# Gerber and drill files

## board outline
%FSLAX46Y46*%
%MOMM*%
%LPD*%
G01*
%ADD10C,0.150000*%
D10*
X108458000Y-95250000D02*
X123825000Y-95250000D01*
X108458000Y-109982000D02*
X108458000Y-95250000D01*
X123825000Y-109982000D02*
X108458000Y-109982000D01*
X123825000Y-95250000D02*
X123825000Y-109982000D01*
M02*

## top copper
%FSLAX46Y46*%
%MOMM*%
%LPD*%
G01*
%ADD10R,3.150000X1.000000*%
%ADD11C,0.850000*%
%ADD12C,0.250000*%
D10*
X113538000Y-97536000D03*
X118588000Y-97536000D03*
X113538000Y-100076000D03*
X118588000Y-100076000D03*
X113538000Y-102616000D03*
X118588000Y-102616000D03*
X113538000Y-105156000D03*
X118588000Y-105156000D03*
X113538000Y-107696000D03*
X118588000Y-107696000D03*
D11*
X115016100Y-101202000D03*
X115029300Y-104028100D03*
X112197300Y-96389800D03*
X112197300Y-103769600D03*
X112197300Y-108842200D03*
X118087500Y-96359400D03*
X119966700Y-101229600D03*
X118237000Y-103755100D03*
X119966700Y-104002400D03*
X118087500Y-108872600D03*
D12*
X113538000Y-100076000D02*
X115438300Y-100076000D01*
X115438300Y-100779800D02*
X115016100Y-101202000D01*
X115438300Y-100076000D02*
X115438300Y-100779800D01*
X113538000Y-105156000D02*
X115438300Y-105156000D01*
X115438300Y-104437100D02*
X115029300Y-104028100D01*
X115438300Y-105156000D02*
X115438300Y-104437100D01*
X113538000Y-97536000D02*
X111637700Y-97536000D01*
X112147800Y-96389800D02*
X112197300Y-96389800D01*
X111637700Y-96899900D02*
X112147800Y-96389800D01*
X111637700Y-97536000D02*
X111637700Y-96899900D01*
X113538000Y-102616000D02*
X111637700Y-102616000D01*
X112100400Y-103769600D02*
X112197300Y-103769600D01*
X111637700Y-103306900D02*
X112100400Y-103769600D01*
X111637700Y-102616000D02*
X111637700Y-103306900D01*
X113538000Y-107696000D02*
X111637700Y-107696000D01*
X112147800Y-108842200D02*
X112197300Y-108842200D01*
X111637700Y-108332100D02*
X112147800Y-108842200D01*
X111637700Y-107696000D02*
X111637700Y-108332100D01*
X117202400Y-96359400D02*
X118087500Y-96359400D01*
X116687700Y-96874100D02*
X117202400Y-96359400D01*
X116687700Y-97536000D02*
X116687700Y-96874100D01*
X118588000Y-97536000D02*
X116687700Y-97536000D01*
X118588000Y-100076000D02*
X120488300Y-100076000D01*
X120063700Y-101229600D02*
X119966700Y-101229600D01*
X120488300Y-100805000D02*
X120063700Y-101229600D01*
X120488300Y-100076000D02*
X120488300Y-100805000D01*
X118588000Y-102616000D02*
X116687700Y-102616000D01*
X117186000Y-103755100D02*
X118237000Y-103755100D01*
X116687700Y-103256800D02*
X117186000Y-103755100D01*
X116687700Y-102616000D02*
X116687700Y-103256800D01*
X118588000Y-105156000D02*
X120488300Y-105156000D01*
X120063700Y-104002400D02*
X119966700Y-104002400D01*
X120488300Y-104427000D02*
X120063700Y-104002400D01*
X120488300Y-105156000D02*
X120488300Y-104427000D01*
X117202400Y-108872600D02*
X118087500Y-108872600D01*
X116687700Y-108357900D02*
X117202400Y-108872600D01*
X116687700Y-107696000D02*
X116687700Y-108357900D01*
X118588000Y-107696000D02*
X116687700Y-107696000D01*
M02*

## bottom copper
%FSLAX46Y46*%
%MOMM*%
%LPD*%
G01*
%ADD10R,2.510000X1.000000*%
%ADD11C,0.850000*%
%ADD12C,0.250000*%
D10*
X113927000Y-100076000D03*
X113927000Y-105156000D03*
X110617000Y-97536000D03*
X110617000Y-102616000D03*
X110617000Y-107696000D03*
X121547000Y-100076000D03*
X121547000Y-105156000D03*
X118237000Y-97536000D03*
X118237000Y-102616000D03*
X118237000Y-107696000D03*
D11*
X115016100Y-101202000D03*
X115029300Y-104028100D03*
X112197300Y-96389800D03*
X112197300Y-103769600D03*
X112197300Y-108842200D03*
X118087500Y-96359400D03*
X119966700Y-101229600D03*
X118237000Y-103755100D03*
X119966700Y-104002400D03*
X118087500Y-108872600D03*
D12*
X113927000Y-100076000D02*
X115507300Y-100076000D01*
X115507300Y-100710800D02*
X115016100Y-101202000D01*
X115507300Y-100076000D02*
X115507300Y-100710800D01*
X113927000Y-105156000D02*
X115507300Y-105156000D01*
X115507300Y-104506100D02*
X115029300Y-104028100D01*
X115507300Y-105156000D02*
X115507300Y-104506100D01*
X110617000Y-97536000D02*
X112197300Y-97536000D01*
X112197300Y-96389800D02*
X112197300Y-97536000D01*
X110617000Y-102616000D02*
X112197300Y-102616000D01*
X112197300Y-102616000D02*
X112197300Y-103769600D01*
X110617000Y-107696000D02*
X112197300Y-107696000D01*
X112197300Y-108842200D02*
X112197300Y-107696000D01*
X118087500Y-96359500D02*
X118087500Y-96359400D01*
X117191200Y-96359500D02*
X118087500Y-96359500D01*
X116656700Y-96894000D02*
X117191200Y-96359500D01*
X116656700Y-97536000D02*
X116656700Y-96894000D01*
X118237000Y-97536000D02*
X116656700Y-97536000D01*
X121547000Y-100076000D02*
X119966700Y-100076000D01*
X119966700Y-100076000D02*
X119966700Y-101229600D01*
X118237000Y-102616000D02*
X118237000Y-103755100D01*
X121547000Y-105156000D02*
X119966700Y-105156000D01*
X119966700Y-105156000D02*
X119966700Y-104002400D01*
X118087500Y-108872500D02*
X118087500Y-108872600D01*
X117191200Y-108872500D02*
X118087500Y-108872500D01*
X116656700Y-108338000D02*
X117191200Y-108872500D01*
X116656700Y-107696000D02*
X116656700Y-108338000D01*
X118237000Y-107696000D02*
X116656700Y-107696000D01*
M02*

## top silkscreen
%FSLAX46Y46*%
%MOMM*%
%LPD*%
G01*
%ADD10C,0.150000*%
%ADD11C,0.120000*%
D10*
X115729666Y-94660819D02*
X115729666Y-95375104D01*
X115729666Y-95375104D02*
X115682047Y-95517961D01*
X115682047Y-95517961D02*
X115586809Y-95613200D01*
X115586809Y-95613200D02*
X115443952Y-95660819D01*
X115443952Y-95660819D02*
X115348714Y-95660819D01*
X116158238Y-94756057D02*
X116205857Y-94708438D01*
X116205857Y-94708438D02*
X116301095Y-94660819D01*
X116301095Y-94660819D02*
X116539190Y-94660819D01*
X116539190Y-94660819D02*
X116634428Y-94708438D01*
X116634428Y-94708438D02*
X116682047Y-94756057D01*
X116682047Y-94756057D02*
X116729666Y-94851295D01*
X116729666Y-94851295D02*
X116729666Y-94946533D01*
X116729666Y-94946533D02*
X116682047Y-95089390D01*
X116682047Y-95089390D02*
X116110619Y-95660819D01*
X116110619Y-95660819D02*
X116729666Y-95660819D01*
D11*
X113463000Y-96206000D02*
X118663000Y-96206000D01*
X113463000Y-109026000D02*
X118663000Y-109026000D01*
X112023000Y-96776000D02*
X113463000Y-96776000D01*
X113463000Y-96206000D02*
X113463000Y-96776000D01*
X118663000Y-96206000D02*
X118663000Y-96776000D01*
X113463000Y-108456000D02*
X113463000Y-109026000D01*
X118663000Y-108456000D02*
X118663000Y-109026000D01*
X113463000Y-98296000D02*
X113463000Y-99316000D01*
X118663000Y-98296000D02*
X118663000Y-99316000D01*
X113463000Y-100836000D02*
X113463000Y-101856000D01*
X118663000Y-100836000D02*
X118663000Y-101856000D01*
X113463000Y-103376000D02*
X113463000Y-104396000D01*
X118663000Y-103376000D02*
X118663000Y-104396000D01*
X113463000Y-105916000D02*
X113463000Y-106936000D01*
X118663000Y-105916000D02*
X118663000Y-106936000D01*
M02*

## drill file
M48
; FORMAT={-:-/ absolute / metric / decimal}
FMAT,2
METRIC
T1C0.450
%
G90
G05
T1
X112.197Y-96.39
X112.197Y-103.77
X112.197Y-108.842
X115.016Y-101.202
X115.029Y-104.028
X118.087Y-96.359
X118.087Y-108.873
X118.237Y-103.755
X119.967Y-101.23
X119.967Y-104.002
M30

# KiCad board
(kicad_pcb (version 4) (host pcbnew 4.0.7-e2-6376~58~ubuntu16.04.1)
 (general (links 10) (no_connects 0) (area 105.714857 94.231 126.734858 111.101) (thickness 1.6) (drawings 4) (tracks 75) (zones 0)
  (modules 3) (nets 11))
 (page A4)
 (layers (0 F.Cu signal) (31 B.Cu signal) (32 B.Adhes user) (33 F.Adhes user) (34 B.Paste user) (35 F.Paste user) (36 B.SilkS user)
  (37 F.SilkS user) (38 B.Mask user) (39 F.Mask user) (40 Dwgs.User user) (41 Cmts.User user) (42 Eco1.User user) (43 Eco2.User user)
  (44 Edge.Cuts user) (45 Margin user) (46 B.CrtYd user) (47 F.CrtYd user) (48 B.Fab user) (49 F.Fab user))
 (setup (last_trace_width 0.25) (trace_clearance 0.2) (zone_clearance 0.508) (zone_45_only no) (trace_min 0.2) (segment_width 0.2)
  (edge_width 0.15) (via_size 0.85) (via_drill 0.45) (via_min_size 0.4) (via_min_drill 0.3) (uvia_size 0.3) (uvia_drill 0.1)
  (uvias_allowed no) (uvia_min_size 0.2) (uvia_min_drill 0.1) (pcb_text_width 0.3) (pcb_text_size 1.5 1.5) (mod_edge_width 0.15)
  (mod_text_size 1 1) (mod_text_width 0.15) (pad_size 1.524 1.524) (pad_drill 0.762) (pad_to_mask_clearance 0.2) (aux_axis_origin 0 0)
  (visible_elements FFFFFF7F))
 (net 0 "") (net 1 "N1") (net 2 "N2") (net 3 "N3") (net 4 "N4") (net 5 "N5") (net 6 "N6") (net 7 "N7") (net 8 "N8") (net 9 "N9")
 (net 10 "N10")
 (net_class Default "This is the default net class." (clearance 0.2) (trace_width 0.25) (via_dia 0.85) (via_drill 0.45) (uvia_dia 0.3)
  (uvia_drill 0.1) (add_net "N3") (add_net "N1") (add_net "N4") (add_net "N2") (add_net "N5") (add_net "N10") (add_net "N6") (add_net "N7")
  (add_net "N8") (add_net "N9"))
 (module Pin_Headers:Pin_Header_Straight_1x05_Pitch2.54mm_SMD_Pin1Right (layer B.Cu) (at 112.272 102.616 180)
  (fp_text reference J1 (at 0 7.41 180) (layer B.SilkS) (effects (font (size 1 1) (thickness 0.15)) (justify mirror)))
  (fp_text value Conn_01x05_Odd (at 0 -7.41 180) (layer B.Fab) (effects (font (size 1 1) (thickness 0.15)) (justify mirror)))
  (pad 2 smd rect (at -1.655 2.54 180) (size 2.51 1) (layers B.Cu B.Paste B.Mask) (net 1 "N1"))
  (pad 4 smd rect (at -1.655 -2.54 180) (size 2.51 1) (layers B.Cu B.Paste B.Mask) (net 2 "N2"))
  (pad 1 smd rect (at 1.655 5.08 180) (size 2.51 1) (layers B.Cu B.Paste B.Mask) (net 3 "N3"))
  (pad 3 smd rect (at 1.655 0 180) (size 2.51 1) (layers B.Cu B.Paste B.Mask) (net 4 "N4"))
  (pad 5 smd rect (at 1.655 -5.08 180) (size 2.51 1) (layers B.Cu B.Paste B.Mask) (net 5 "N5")))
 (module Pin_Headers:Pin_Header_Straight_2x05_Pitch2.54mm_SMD (layer F.Cu) (at 116.063 102.616)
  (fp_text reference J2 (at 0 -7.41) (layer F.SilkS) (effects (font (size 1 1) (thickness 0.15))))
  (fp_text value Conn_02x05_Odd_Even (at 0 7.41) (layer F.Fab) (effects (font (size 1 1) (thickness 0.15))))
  (fp_line (start -2.6 -6.41) (end 2.6 -6.41) (layer F.SilkS) (width 0.12))
  (fp_line (start -2.6 6.41) (end 2.6 6.41) (layer F.SilkS) (width 0.12))
  (fp_line (start -4.04 -5.84) (end -2.6 -5.84) (layer F.SilkS) (width 0.12))
  (fp_line (start -2.6 -6.41) (end -2.6 -5.84) (layer F.SilkS) (width 0.12))
  (fp_line (start 2.6 -6.41) (end 2.6 -5.84) (layer F.SilkS) (width 0.12))
  (fp_line (start -2.6 5.84) (end -2.6 6.41) (layer F.SilkS) (width 0.12))
  (fp_line (start 2.6 5.84) (end 2.6 6.41) (layer F.SilkS) (width 0.12))
  (fp_line (start -2.6 -4.32) (end -2.6 -3.3) (layer F.SilkS) (width 0.12))
  (fp_line (start 2.6 -4.32) (end 2.6 -3.3) (layer F.SilkS) (width 0.12))
  (fp_line (start -2.6 -1.78) (end -2.6 -0.76) (layer F.SilkS) (width 0.12))
  (fp_line (start 2.6 -1.78) (end 2.6 -0.76) (layer F.SilkS) (width 0.12))
  (fp_line (start -2.6 0.76) (end -2.6 1.78) (layer F.SilkS) (width 0.12))
  (fp_line (start 2.6 0.76) (end 2.6 1.78) (layer F.SilkS) (width 0.12))
  (fp_line (start -2.6 3.3) (end -2.6 4.32) (layer F.SilkS) (width 0.12))
  (fp_line (start 2.6 3.3) (end 2.6 4.32) (layer F.SilkS) (width 0.12))
  (pad 1 smd rect (at -2.525 -5.08) (size 3.15 1) (layers F.Cu F.Paste F.Mask) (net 3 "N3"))
  (pad 2 smd rect (at 2.525 -5.08) (size 3.15 1) (layers F.Cu F.Paste F.Mask) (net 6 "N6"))
  (pad 3 smd rect (at -2.525 -2.54) (size 3.15 1) (layers F.Cu F.Paste F.Mask) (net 1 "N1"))
  (pad 4 smd rect (at 2.525 -2.54) (size 3.15 1) (layers F.Cu F.Paste F.Mask) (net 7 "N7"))
  (pad 5 smd rect (at -2.525 0) (size 3.15 1) (layers F.Cu F.Paste F.Mask) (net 4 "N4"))
  (pad 6 smd rect (at 2.525 0) (size 3.15 1) (layers F.Cu F.Paste F.Mask) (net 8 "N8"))
  (pad 7 smd rect (at -2.525 2.54) (size 3.15 1) (layers F.Cu F.Paste F.Mask) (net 2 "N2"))
  (pad 8 smd rect (at 2.525 2.54) (size 3.15 1) (layers F.Cu F.Paste F.Mask) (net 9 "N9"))
  (pad 9 smd rect (at -2.525 5.08) (size 3.15 1) (layers F.Cu F.Paste F.Mask) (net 5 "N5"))
  (pad 10 smd rect (at 2.525 5.08) (size 3.15 1) (layers F.Cu F.Paste F.Mask) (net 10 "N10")))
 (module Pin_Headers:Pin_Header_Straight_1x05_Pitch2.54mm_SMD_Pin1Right (layer B.Cu) (at 119.892 102.616 180)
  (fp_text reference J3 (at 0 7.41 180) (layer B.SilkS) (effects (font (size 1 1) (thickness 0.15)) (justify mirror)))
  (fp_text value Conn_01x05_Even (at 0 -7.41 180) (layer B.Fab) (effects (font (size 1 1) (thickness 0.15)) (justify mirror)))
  (pad 2 smd rect (at -1.655 2.54 180) (size 2.51 1) (layers B.Cu B.Paste B.Mask) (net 7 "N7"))
  (pad 4 smd rect (at -1.655 -2.54 180) (size 2.51 1) (layers B.Cu B.Paste B.Mask) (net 9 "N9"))
  (pad 1 smd rect (at 1.655 5.08 180) (size 2.51 1) (layers B.Cu B.Paste B.Mask) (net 6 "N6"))
  (pad 3 smd rect (at 1.655 0 180) (size 2.51 1) (layers B.Cu B.Paste B.Mask) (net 8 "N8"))
  (pad 5 smd rect (at 1.655 -5.08 180) (size 2.51 1) (layers B.Cu B.Paste B.Mask) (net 10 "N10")))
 (gr_line (start 108.458 95.25) (end 123.825 95.25) (layer Edge.Cuts) (width 0.15))
 (gr_line (start 108.458 109.982) (end 108.458 95.25) (layer Edge.Cuts) (width 0.15))
 (gr_line (start 123.825 109.982) (end 108.458 109.982) (layer Edge.Cuts) (width 0.15))
 (gr_line (start 123.825 95.25) (end 123.825 109.982) (layer Edge.Cuts) (width 0.15))
 (via (at 115.0161 101.202) (size 0.85) (layers F.Cu B.Cu) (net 1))
 (segment (start 113.538 100.076) (end 115.4383 100.076) (width 0.25) (layer F.Cu) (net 1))
 (segment (start 113.927 100.076) (end 115.5073 100.076) (width 0.25) (layer B.Cu) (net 1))
 (segment (start 115.5073 100.7108) (end 115.0161 101.202) (width 0.25) (layer B.Cu) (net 1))
 (segment (start 115.5073 100.076) (end 115.5073 100.7108) (width 0.25) (layer B.Cu) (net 1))
 (segment (start 115.4383 100.7798) (end 115.0161 101.202) (width 0.25) (layer F.Cu) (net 1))
 (segment (start 115.4383 100.076) (end 115.4383 100.7798) (width 0.25) (layer F.Cu) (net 1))
 (via (at 115.0293 104.0281) (size 0.85) (layers F.Cu B.Cu) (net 2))
 (segment (start 113.538 105.156) (end 115.4383 105.156) (width 0.25) (layer F.Cu) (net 2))
 (segment (start 113.927 105.156) (end 115.5073 105.156) (width 0.25) (layer B.Cu) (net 2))
 (segment (start 115.5073 104.5061) (end 115.0293 104.0281) (width 0.25) (layer B.Cu) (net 2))
 (segment (start 115.5073 105.156) (end 115.5073 104.5061) (width 0.25) (layer B.Cu) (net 2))
 (segment (start 115.4383 104.4371) (end 115.0293 104.0281) (width 0.25) (layer F.Cu) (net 2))
 (segment (start 115.4383 105.156) (end 115.4383 104.4371) (width 0.25) (layer F.Cu) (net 2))
 (via (at 112.1973 96.3898) (size 0.85) (layers F.Cu B.Cu) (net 3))
 (segment (start 110.617 97.536) (end 112.1973 97.536) (width 0.25) (layer B.Cu) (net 3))
 (segment (start 113.538 97.536) (end 111.6377 97.536) (width 0.25) (layer F.Cu) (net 3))
 (segment (start 112.1973 96.3898) (end 112.1973 97.536) (width 0.25) (layer B.Cu) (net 3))
 (segment (start 112.1478 96.3898) (end 112.1973 96.3898) (width 0.25) (layer F.Cu) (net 3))
 (segment (start 111.6377 96.8999) (end 112.1478 96.3898) (width 0.25) (layer F.Cu) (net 3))
 (segment (start 111.6377 97.536) (end 111.6377 96.8999) (width 0.25) (layer F.Cu) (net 3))
 (via (at 112.1973 103.7696) (size 0.85) (layers F.Cu B.Cu) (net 4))
 (segment (start 110.617 102.616) (end 112.1973 102.616) (width 0.25) (layer B.Cu) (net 4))
 (segment (start 113.538 102.616) (end 111.6377 102.616) (width 0.25) (layer F.Cu) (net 4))
 (segment (start 112.1973 102.616) (end 112.1973 103.7696) (width 0.25) (layer B.Cu) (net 4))
 (segment (start 112.1004 103.7696) (end 112.1973 103.7696) (width 0.25) (layer F.Cu) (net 4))
 (segment (start 111.6377 103.3069) (end 112.1004 103.7696) (width 0.25) (layer F.Cu) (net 4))
 (segment (start 111.6377 102.616) (end 111.6377 103.3069) (width 0.25) (layer F.Cu) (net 4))
 (via (at 112.1973 108.8422) (size 0.85) (layers F.Cu B.Cu) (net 5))
 (segment (start 110.617 107.696) (end 112.1973 107.696) (width 0.25) (layer B.Cu) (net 5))
 (segment (start 113.538 107.696) (end 111.6377 107.696) (width 0.25) (layer F.Cu) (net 5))
 (segment (start 112.1973 108.8422) (end 112.1973 107.696) (width 0.25) (layer B.Cu) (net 5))
 (segment (start 112.1478 108.8422) (end 112.1973 108.8422) (width 0.25) (layer F.Cu) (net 5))
 (segment (start 111.6377 108.3321) (end 112.1478 108.8422) (width 0.25) (layer F.Cu) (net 5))
 (segment (start 111.6377 107.696) (end 111.6377 108.3321) (width 0.25) (layer F.Cu) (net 5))
 (via (at 118.0875 96.3594) (size 0.85) (layers F.Cu B.Cu) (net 6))
 (segment (start 118.0875 96.3595) (end 118.0875 96.3594) (width 0.25) (layer B.Cu) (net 6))
 (segment (start 117.1912 96.3595) (end 118.0875 96.3595) (width 0.25) (layer B.Cu) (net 6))
 (segment (start 116.6567 96.894) (end 117.1912 96.3595) (width 0.25) (layer B.Cu) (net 6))
 (segment (start 116.6567 97.536) (end 116.6567 96.894) (width 0.25) (layer B.Cu) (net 6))
 (segment (start 117.2024 96.3594) (end 118.0875 96.3594) (width 0.25) (layer F.Cu) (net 6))
 (segment (start 116.6877 96.8741) (end 117.2024 96.3594) (width 0.25) (layer F.Cu) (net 6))
 (segment (start 116.6877 97.536) (end 116.6877 96.8741) (width 0.25) (layer F.Cu) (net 6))
 (segment (start 118.588 97.536) (end 116.6877 97.536) (width 0.25) (layer F.Cu) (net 6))
 (segment (start 118.237 97.536) (end 116.6567 97.536) (width 0.25) (layer B.Cu) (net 6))
 (via (at 119.9667 101.2296) (size 0.85) (layers F.Cu B.Cu) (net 7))
 (segment (start 121.547 100.076) (end 119.9667 100.076) (width 0.25) (layer B.Cu) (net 7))
 (segment (start 118.588 100.076) (end 120.4883 100.076) (width 0.25) (layer F.Cu) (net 7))
 (segment (start 119.9667 100.076) (end 119.9667 101.2296) (width 0.25) (layer B.Cu) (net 7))
 (segment (start 120.0637 101.2296) (end 119.9667 101.2296) (width 0.25) (layer F.Cu) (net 7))
 (segment (start 120.4883 100.805) (end 120.0637 101.2296) (width 0.25) (layer F.Cu) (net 7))
 (segment (start 120.4883 100.076) (end 120.4883 100.805) (width 0.25) (layer F.Cu) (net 7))
 (via (at 118.237 103.7551) (size 0.85) (layers F.Cu B.Cu) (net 8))
 (segment (start 118.588 102.616) (end 116.6877 102.616) (width 0.25) (layer F.Cu) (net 8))
 (segment (start 118.237 102.616) (end 118.237 103.7551) (width 0.25) (layer B.Cu) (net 8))
 (segment (start 117.186 103.7551) (end 118.237 103.7551) (width 0.25) (layer F.Cu) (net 8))
 (segment (start 116.6877 103.2568) (end 117.186 103.7551) (width 0.25) (layer F.Cu) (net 8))
 (segment (start 116.6877 102.616) (end 116.6877 103.2568) (width 0.25) (layer F.Cu) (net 8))
 (via (at 119.9667 104.0024) (size 0.85) (layers F.Cu B.Cu) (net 9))
 (segment (start 121.547 105.156) (end 119.9667 105.156) (width 0.25) (layer B.Cu) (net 9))
 (segment (start 118.588 105.156) (end 120.4883 105.156) (width 0.25) (layer F.Cu) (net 9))
 (segment (start 119.9667 105.156) (end 119.9667 104.0024) (width 0.25) (layer B.Cu) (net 9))
 (segment (start 120.0637 104.0024) (end 119.9667 104.0024) (width 0.25) (layer F.Cu) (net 9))
 (segment (start 120.4883 104.427) (end 120.0637 104.0024) (width 0.25) (layer F.Cu) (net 9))
 (segment (start 120.4883 105.156) (end 120.4883 104.427) (width 0.25) (layer F.Cu) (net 9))
 (via (at 118.0875 108.8726) (size 0.85) (layers F.Cu B.Cu) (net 10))
 (segment (start 118.0875 108.8725) (end 118.0875 108.8726) (width 0.25) (layer B.Cu) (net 10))
 (segment (start 117.1912 108.8725) (end 118.0875 108.8725) (width 0.25) (layer B.Cu) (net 10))
 (segment (start 116.6567 108.338) (end 117.1912 108.8725) (width 0.25) (layer B.Cu) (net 10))
 (segment (start 116.6567 107.696) (end 116.6567 108.338) (width 0.25) (layer B.Cu) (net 10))
 (segment (start 117.2024 108.8726) (end 118.0875 108.8726) (width 0.25) (layer F.Cu) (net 10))
 (segment (start 116.6877 108.3579) (end 117.2024 108.8726) (width 0.25) (layer F.Cu) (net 10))
 (segment (start 116.6877 107.696) (end 116.6877 108.3579) (width 0.25) (layer F.Cu) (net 10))
 (segment (start 118.588 107.696) (end 116.6877 107.696) (width 0.25) (layer F.Cu) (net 10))
 (segment (start 118.237 107.696) (end 116.6567 107.696) (width 0.25) (layer B.Cu) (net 10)))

